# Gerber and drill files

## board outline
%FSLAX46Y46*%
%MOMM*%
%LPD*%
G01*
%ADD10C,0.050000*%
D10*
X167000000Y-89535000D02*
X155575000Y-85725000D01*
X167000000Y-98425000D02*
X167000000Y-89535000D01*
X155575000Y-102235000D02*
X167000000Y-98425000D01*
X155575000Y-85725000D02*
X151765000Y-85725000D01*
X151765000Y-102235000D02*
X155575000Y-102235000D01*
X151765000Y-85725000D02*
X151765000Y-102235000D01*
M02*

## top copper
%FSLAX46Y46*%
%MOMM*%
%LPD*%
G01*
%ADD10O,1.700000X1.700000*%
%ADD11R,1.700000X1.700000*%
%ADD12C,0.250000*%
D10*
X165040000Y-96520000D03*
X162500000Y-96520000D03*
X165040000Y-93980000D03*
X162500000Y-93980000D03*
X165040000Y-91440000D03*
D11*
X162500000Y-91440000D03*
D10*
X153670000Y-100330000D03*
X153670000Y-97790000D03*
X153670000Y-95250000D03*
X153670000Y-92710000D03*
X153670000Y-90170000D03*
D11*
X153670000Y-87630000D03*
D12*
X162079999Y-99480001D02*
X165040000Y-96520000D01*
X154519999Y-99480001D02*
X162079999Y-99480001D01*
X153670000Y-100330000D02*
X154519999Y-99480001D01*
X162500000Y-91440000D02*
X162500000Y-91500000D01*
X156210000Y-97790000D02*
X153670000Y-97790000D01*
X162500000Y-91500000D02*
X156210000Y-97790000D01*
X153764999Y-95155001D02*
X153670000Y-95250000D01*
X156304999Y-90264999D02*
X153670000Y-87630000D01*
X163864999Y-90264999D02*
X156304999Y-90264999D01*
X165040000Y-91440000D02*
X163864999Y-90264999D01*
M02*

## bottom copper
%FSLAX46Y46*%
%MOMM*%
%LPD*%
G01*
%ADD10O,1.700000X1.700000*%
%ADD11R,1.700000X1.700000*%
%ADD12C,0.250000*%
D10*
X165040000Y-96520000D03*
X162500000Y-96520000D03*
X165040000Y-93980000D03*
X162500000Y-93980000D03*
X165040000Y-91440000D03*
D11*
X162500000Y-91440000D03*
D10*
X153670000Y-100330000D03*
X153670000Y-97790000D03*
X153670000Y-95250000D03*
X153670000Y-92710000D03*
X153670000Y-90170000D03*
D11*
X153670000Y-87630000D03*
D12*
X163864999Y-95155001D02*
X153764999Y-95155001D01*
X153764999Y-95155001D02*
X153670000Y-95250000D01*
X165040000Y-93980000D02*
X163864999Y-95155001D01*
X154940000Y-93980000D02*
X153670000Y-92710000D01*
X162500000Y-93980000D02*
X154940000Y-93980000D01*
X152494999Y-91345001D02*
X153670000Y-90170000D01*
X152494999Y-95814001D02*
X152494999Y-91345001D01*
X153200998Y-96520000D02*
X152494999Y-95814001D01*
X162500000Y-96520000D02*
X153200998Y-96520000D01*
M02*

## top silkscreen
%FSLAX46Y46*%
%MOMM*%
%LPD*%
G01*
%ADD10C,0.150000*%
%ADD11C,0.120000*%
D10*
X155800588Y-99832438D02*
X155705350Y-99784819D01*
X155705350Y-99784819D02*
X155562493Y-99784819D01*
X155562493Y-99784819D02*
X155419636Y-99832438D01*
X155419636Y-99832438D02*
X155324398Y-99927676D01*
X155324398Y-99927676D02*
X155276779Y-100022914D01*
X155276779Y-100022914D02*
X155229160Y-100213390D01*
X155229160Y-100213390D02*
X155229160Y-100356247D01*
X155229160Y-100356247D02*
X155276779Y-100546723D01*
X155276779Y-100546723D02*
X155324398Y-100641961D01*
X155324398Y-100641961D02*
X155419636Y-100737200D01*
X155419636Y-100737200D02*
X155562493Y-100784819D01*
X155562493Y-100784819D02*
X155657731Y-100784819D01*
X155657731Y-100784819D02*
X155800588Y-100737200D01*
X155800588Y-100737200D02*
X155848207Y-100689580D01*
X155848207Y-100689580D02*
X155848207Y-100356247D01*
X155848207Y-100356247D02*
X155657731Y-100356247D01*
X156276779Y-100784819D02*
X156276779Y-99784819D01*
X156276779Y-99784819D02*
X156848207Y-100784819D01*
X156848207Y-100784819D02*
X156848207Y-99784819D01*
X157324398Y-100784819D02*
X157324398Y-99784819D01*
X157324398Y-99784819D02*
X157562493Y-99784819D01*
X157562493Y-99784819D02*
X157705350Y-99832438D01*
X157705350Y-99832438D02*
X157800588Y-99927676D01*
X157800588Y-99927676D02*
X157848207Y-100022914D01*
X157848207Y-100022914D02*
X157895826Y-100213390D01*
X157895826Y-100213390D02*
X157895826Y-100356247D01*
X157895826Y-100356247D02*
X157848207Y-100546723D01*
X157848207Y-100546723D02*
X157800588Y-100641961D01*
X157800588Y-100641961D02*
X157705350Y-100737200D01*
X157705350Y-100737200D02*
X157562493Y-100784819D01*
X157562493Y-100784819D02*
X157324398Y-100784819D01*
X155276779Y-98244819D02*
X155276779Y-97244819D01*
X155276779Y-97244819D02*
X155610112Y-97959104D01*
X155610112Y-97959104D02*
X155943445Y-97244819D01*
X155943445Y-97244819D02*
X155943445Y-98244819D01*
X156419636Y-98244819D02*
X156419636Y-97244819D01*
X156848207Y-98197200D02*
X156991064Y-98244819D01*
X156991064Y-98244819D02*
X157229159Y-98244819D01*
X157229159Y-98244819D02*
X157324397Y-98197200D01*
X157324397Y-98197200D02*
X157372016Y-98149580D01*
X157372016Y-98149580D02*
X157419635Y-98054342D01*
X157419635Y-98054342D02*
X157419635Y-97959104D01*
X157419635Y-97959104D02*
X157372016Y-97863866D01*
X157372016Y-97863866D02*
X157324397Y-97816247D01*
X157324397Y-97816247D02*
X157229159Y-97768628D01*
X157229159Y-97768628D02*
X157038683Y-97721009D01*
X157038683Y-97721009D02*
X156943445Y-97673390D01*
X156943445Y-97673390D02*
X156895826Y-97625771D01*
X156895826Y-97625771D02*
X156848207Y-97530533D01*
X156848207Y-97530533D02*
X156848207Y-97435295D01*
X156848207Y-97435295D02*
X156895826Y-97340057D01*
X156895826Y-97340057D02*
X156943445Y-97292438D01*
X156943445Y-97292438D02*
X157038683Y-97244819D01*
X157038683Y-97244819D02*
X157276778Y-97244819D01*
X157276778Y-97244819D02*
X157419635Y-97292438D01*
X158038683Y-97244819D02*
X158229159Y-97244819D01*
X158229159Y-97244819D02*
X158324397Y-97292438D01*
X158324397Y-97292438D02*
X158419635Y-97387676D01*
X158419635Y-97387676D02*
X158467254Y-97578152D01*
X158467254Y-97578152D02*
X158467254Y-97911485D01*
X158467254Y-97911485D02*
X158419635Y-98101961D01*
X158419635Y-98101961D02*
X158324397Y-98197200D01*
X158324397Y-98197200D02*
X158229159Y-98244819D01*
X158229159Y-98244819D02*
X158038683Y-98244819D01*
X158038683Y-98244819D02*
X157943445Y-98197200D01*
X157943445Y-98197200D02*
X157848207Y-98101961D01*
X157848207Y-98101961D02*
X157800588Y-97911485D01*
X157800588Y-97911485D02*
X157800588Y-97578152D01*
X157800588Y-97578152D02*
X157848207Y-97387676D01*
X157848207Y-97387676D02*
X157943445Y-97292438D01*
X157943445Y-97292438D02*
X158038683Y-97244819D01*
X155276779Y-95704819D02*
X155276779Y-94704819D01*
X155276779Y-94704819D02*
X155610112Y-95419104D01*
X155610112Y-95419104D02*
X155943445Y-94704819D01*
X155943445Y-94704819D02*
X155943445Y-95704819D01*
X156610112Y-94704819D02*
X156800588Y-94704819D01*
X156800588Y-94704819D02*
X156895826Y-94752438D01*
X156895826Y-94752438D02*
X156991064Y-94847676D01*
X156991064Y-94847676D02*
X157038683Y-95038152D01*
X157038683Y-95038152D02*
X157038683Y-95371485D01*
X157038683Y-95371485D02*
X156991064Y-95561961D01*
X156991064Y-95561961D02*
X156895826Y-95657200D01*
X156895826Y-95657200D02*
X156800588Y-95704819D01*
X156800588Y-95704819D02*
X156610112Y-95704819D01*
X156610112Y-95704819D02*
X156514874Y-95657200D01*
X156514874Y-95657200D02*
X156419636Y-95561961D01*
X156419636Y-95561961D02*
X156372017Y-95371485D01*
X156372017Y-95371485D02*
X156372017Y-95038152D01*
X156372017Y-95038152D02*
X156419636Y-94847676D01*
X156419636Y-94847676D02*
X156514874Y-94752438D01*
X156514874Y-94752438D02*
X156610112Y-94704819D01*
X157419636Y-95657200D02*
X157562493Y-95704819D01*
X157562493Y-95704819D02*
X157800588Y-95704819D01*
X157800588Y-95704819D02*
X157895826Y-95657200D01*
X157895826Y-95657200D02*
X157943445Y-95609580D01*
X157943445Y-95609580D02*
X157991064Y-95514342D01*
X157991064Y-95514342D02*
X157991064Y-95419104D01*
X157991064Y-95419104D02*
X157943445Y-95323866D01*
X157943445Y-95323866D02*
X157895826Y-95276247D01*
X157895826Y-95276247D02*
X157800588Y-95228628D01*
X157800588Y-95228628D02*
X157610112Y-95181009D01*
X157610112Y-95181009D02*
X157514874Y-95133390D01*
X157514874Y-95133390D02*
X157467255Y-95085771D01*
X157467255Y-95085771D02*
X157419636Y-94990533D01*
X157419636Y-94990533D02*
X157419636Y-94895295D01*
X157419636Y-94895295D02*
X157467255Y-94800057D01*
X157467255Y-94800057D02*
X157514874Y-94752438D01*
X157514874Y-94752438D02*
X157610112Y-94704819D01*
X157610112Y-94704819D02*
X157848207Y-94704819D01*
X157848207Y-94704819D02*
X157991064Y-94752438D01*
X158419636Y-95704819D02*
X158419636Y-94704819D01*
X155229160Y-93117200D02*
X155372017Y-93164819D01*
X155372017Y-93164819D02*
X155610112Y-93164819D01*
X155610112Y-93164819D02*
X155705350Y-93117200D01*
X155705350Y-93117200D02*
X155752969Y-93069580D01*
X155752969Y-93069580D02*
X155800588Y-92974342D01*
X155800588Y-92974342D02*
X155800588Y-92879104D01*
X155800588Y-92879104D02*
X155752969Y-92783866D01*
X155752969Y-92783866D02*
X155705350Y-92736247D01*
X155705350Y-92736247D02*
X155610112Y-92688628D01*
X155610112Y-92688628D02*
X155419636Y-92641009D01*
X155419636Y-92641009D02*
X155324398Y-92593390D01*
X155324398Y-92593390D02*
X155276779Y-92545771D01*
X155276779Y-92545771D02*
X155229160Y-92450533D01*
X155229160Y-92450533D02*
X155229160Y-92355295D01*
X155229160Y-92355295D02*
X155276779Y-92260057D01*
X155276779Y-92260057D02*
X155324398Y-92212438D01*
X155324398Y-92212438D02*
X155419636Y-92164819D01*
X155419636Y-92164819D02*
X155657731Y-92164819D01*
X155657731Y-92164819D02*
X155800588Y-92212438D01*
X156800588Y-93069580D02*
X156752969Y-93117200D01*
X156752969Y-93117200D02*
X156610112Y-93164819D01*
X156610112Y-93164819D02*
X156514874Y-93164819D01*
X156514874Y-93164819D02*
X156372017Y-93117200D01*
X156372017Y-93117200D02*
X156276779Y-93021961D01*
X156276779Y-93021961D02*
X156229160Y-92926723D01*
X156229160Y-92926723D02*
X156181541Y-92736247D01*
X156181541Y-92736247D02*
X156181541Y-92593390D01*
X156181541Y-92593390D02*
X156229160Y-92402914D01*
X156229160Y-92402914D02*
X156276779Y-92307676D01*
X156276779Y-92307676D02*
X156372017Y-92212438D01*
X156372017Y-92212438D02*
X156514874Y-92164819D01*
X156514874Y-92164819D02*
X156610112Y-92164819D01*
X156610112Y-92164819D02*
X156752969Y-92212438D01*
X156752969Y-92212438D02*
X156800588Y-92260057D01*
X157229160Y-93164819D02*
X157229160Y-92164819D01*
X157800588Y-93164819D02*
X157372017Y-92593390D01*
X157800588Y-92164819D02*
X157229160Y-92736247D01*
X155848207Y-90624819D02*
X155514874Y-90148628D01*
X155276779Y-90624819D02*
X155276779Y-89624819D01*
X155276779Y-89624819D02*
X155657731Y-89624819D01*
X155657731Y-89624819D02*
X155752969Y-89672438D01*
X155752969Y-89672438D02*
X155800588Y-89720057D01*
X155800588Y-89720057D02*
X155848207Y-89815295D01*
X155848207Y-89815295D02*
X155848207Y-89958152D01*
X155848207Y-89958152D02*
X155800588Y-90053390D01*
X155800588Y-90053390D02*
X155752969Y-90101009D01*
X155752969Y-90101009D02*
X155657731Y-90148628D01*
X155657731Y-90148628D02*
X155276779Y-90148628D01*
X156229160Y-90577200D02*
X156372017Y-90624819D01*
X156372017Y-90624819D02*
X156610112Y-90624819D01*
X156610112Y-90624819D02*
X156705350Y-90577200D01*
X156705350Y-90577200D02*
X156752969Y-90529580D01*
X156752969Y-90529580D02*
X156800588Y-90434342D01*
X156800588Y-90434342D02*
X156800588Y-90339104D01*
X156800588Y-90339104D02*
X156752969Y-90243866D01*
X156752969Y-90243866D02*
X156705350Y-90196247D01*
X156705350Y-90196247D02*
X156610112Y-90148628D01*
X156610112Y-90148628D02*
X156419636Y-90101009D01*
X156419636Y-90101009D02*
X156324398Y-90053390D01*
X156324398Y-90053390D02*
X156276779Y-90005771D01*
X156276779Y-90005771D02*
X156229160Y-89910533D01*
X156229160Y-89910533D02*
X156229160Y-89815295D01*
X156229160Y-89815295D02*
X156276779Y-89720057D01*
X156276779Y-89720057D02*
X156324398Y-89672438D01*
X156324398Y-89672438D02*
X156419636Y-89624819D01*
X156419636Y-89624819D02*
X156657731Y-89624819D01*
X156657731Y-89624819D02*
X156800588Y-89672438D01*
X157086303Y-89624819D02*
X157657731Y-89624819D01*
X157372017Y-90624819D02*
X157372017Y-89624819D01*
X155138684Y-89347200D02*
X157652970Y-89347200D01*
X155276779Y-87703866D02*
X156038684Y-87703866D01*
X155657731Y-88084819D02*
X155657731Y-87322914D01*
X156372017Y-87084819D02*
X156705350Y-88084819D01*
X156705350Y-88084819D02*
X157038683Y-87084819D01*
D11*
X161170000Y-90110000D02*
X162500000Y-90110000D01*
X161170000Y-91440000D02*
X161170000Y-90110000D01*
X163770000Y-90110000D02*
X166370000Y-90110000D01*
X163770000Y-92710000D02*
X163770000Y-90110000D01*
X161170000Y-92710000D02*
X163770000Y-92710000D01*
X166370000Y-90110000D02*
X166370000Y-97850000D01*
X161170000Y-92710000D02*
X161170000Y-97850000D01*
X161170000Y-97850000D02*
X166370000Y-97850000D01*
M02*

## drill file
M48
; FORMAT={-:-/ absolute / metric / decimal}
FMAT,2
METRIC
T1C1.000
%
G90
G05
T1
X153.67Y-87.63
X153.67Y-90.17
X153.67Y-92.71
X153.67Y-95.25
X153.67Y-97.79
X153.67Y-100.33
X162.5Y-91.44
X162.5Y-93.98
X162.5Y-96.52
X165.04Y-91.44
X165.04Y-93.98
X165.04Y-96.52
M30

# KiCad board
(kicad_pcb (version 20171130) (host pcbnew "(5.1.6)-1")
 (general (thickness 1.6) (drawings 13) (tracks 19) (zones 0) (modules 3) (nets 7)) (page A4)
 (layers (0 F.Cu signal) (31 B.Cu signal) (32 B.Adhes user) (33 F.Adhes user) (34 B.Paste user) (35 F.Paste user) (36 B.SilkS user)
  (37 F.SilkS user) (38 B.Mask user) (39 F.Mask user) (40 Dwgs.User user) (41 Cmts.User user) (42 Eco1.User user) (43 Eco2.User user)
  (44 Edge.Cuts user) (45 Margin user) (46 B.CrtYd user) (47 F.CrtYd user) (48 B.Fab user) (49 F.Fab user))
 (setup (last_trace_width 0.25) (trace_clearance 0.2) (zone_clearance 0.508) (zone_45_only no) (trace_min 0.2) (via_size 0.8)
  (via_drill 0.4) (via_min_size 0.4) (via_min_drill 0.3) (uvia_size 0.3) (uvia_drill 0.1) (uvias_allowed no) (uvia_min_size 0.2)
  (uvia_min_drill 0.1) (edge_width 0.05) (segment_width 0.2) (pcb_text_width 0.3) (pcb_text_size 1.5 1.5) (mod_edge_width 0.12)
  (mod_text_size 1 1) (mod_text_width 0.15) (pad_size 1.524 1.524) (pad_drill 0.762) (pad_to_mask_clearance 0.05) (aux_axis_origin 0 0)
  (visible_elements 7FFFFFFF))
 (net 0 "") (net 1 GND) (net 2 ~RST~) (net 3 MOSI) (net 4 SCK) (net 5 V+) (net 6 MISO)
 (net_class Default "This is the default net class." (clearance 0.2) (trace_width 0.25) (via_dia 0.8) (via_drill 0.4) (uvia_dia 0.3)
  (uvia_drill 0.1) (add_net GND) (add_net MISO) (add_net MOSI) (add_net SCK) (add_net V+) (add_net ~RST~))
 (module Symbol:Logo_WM (layer B.Cu) (at 158 90.1 270)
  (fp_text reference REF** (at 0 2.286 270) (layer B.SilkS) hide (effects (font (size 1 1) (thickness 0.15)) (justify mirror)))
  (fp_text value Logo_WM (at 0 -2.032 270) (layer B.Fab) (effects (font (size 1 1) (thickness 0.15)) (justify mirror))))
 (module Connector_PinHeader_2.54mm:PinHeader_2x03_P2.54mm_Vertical (layer F.Cu) (at 162.5 91.44)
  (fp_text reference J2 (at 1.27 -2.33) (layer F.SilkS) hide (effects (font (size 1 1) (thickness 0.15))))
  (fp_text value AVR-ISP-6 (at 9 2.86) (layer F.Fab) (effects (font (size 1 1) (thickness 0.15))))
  (fp_line (start -1.33 -1.33) (end 0 -1.33) (layer F.SilkS) (width 0.12))
  (fp_line (start -1.33 0) (end -1.33 -1.33) (layer F.SilkS) (width 0.12))
  (fp_line (start 1.27 -1.33) (end 3.87 -1.33) (layer F.SilkS) (width 0.12))
  (fp_line (start 1.27 1.27) (end 1.27 -1.33) (layer F.SilkS) (width 0.12))
  (fp_line (start -1.33 1.27) (end 1.27 1.27) (layer F.SilkS) (width 0.12))
  (fp_line (start 3.87 -1.33) (end 3.87 6.41) (layer F.SilkS) (width 0.12))
  (fp_line (start -1.33 1.27) (end -1.33 6.41) (layer F.SilkS) (width 0.12))
  (fp_line (start -1.33 6.41) (end 3.87 6.41) (layer F.SilkS) (width 0.12))
  (pad 6 thru_hole oval (at 2.54 5.08) (size 1.7 1.7) (drill 1) (layers *.Cu *.Mask) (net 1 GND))
  (pad 5 thru_hole oval (at 0 5.08) (size 1.7 1.7) (drill 1) (layers *.Cu *.Mask) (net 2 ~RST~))
  (pad 4 thru_hole oval (at 2.54 2.54) (size 1.7 1.7) (drill 1) (layers *.Cu *.Mask) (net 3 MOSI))
  (pad 3 thru_hole oval (at 0 2.54) (size 1.7 1.7) (drill 1) (layers *.Cu *.Mask) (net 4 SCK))
  (pad 2 thru_hole oval (at 2.54 0) (size 1.7 1.7) (drill 1) (layers *.Cu *.Mask) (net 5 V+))
  (pad 1 thru_hole rect (at 0 0) (size 1.7 1.7) (drill 1) (layers *.Cu *.Mask) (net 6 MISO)))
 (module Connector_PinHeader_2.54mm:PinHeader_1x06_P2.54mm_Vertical (layer B.Cu) (at 153.67 87.63 180)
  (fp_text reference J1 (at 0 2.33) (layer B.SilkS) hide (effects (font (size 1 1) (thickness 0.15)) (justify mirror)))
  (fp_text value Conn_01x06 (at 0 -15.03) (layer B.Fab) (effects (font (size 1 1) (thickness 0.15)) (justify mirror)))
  (pad 6 thru_hole oval (at 0 -12.7 180) (size 1.7 1.7) (drill 1) (layers *.Cu *.Mask) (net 1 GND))
  (pad 5 thru_hole oval (at 0 -10.16 180) (size 1.7 1.7) (drill 1) (layers *.Cu *.Mask) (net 6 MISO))
  (pad 4 thru_hole oval (at 0 -7.62 180) (size 1.7 1.7) (drill 1) (layers *.Cu *.Mask) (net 3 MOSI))
  (pad 3 thru_hole oval (at 0 -5.08 180) (size 1.7 1.7) (drill 1) (layers *.Cu *.Mask) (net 4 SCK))
  (pad 2 thru_hole oval (at 0 -2.54 180) (size 1.7 1.7) (drill 1) (layers *.Cu *.Mask) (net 2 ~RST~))
  (pad 1 thru_hole rect (at 0 0 180) (size 1.7 1.7) (drill 1) (layers *.Cu *.Mask) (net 5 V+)))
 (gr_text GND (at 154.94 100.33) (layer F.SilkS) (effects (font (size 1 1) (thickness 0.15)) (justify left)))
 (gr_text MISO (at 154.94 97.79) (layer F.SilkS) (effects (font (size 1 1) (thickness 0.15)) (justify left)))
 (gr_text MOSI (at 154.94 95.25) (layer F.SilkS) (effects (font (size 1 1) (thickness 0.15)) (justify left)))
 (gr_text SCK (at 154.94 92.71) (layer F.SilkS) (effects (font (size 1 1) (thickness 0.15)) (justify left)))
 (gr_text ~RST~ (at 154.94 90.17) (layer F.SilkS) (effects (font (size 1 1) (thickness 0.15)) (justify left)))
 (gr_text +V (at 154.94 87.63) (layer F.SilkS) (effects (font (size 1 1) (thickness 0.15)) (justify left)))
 (gr_line (start 167 89.535) (end 155.575 85.725) (layer Edge.Cuts) (width 0.05))
 (gr_line (start 167 98.425) (end 167 89.535) (layer Edge.Cuts) (width 0.05))
 (gr_line (start 155.575 102.235) (end 167 98.425) (layer Edge.Cuts) (width 0.05))
 (gr_line (start 155.575 85.725) (end 151.765 85.725) (layer Edge.Cuts) (width 0.05))
 (gr_line (start 151.765 102.235) (end 155.575 102.235) (layer Edge.Cuts) (width 0.05))
 (gr_line (start 151.765 85.725) (end 151.765 102.235) (layer Edge.Cuts) (width 0.05))
 (segment (start 162.079999 99.480001) (end 165.04 96.52) (width 0.25) (layer F.Cu) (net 1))
 (segment (start 154.519999 99.480001) (end 162.079999 99.480001) (width 0.25) (layer F.Cu) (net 1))
 (segment (start 153.67 100.33) (end 154.519999 99.480001) (width 0.25) (layer F.Cu) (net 1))
 (segment (start 162.5 91.44) (end 162.5 91.5) (width 0.25) (layer F.Cu) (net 6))
 (segment (start 156.21 97.79) (end 153.67 97.79) (width 0.25) (layer F.Cu) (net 6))
 (segment (start 162.5 91.5) (end 156.21 97.79) (width 0.25) (layer F.Cu) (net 6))
 (segment (start 153.764999 95.155001) (end 153.67 95.25) (width 0.25) (layer F.Cu) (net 3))
 (segment (start 163.864999 95.155001) (end 153.764999 95.155001) (width 0.25) (layer B.Cu) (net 3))
 (segment (start 153.764999 95.155001) (end 153.67 95.25) (width 0.25) (layer B.Cu) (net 3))
 (segment (start 165.04 93.98) (end 163.864999 95.155001) (width 0.25) (layer B.Cu) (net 3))
 (segment (start 154.94 93.98) (end 153.67 92.71) (width 0.25) (layer B.Cu) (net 4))
 (segment (start 162.5 93.98) (end 154.94 93.98) (width 0.25) (layer B.Cu) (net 4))
 (segment (start 152.494999 91.345001) (end 153.67 90.17) (width 0.25) (layer B.Cu) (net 2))
 (segment (start 152.494999 95.814001) (end 152.494999 91.345001) (width 0.25) (layer B.Cu) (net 2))
 (segment (start 153.200998 96.52) (end 152.494999 95.814001) (width 0.25) (layer B.Cu) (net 2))
 (segment (start 162.5 96.52) (end 153.200998 96.52) (width 0.25) (layer B.Cu) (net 2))
 (segment (start 156.304999 90.264999) (end 153.67 87.63) (width 0.25) (layer F.Cu) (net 5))
 (segment (start 163.864999 90.264999) (end 156.304999 90.264999) (width 0.25) (layer F.Cu) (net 5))
 (segment (start 165.04 91.44) (end 163.864999 90.264999) (width 0.25) (layer F.Cu) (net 5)))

